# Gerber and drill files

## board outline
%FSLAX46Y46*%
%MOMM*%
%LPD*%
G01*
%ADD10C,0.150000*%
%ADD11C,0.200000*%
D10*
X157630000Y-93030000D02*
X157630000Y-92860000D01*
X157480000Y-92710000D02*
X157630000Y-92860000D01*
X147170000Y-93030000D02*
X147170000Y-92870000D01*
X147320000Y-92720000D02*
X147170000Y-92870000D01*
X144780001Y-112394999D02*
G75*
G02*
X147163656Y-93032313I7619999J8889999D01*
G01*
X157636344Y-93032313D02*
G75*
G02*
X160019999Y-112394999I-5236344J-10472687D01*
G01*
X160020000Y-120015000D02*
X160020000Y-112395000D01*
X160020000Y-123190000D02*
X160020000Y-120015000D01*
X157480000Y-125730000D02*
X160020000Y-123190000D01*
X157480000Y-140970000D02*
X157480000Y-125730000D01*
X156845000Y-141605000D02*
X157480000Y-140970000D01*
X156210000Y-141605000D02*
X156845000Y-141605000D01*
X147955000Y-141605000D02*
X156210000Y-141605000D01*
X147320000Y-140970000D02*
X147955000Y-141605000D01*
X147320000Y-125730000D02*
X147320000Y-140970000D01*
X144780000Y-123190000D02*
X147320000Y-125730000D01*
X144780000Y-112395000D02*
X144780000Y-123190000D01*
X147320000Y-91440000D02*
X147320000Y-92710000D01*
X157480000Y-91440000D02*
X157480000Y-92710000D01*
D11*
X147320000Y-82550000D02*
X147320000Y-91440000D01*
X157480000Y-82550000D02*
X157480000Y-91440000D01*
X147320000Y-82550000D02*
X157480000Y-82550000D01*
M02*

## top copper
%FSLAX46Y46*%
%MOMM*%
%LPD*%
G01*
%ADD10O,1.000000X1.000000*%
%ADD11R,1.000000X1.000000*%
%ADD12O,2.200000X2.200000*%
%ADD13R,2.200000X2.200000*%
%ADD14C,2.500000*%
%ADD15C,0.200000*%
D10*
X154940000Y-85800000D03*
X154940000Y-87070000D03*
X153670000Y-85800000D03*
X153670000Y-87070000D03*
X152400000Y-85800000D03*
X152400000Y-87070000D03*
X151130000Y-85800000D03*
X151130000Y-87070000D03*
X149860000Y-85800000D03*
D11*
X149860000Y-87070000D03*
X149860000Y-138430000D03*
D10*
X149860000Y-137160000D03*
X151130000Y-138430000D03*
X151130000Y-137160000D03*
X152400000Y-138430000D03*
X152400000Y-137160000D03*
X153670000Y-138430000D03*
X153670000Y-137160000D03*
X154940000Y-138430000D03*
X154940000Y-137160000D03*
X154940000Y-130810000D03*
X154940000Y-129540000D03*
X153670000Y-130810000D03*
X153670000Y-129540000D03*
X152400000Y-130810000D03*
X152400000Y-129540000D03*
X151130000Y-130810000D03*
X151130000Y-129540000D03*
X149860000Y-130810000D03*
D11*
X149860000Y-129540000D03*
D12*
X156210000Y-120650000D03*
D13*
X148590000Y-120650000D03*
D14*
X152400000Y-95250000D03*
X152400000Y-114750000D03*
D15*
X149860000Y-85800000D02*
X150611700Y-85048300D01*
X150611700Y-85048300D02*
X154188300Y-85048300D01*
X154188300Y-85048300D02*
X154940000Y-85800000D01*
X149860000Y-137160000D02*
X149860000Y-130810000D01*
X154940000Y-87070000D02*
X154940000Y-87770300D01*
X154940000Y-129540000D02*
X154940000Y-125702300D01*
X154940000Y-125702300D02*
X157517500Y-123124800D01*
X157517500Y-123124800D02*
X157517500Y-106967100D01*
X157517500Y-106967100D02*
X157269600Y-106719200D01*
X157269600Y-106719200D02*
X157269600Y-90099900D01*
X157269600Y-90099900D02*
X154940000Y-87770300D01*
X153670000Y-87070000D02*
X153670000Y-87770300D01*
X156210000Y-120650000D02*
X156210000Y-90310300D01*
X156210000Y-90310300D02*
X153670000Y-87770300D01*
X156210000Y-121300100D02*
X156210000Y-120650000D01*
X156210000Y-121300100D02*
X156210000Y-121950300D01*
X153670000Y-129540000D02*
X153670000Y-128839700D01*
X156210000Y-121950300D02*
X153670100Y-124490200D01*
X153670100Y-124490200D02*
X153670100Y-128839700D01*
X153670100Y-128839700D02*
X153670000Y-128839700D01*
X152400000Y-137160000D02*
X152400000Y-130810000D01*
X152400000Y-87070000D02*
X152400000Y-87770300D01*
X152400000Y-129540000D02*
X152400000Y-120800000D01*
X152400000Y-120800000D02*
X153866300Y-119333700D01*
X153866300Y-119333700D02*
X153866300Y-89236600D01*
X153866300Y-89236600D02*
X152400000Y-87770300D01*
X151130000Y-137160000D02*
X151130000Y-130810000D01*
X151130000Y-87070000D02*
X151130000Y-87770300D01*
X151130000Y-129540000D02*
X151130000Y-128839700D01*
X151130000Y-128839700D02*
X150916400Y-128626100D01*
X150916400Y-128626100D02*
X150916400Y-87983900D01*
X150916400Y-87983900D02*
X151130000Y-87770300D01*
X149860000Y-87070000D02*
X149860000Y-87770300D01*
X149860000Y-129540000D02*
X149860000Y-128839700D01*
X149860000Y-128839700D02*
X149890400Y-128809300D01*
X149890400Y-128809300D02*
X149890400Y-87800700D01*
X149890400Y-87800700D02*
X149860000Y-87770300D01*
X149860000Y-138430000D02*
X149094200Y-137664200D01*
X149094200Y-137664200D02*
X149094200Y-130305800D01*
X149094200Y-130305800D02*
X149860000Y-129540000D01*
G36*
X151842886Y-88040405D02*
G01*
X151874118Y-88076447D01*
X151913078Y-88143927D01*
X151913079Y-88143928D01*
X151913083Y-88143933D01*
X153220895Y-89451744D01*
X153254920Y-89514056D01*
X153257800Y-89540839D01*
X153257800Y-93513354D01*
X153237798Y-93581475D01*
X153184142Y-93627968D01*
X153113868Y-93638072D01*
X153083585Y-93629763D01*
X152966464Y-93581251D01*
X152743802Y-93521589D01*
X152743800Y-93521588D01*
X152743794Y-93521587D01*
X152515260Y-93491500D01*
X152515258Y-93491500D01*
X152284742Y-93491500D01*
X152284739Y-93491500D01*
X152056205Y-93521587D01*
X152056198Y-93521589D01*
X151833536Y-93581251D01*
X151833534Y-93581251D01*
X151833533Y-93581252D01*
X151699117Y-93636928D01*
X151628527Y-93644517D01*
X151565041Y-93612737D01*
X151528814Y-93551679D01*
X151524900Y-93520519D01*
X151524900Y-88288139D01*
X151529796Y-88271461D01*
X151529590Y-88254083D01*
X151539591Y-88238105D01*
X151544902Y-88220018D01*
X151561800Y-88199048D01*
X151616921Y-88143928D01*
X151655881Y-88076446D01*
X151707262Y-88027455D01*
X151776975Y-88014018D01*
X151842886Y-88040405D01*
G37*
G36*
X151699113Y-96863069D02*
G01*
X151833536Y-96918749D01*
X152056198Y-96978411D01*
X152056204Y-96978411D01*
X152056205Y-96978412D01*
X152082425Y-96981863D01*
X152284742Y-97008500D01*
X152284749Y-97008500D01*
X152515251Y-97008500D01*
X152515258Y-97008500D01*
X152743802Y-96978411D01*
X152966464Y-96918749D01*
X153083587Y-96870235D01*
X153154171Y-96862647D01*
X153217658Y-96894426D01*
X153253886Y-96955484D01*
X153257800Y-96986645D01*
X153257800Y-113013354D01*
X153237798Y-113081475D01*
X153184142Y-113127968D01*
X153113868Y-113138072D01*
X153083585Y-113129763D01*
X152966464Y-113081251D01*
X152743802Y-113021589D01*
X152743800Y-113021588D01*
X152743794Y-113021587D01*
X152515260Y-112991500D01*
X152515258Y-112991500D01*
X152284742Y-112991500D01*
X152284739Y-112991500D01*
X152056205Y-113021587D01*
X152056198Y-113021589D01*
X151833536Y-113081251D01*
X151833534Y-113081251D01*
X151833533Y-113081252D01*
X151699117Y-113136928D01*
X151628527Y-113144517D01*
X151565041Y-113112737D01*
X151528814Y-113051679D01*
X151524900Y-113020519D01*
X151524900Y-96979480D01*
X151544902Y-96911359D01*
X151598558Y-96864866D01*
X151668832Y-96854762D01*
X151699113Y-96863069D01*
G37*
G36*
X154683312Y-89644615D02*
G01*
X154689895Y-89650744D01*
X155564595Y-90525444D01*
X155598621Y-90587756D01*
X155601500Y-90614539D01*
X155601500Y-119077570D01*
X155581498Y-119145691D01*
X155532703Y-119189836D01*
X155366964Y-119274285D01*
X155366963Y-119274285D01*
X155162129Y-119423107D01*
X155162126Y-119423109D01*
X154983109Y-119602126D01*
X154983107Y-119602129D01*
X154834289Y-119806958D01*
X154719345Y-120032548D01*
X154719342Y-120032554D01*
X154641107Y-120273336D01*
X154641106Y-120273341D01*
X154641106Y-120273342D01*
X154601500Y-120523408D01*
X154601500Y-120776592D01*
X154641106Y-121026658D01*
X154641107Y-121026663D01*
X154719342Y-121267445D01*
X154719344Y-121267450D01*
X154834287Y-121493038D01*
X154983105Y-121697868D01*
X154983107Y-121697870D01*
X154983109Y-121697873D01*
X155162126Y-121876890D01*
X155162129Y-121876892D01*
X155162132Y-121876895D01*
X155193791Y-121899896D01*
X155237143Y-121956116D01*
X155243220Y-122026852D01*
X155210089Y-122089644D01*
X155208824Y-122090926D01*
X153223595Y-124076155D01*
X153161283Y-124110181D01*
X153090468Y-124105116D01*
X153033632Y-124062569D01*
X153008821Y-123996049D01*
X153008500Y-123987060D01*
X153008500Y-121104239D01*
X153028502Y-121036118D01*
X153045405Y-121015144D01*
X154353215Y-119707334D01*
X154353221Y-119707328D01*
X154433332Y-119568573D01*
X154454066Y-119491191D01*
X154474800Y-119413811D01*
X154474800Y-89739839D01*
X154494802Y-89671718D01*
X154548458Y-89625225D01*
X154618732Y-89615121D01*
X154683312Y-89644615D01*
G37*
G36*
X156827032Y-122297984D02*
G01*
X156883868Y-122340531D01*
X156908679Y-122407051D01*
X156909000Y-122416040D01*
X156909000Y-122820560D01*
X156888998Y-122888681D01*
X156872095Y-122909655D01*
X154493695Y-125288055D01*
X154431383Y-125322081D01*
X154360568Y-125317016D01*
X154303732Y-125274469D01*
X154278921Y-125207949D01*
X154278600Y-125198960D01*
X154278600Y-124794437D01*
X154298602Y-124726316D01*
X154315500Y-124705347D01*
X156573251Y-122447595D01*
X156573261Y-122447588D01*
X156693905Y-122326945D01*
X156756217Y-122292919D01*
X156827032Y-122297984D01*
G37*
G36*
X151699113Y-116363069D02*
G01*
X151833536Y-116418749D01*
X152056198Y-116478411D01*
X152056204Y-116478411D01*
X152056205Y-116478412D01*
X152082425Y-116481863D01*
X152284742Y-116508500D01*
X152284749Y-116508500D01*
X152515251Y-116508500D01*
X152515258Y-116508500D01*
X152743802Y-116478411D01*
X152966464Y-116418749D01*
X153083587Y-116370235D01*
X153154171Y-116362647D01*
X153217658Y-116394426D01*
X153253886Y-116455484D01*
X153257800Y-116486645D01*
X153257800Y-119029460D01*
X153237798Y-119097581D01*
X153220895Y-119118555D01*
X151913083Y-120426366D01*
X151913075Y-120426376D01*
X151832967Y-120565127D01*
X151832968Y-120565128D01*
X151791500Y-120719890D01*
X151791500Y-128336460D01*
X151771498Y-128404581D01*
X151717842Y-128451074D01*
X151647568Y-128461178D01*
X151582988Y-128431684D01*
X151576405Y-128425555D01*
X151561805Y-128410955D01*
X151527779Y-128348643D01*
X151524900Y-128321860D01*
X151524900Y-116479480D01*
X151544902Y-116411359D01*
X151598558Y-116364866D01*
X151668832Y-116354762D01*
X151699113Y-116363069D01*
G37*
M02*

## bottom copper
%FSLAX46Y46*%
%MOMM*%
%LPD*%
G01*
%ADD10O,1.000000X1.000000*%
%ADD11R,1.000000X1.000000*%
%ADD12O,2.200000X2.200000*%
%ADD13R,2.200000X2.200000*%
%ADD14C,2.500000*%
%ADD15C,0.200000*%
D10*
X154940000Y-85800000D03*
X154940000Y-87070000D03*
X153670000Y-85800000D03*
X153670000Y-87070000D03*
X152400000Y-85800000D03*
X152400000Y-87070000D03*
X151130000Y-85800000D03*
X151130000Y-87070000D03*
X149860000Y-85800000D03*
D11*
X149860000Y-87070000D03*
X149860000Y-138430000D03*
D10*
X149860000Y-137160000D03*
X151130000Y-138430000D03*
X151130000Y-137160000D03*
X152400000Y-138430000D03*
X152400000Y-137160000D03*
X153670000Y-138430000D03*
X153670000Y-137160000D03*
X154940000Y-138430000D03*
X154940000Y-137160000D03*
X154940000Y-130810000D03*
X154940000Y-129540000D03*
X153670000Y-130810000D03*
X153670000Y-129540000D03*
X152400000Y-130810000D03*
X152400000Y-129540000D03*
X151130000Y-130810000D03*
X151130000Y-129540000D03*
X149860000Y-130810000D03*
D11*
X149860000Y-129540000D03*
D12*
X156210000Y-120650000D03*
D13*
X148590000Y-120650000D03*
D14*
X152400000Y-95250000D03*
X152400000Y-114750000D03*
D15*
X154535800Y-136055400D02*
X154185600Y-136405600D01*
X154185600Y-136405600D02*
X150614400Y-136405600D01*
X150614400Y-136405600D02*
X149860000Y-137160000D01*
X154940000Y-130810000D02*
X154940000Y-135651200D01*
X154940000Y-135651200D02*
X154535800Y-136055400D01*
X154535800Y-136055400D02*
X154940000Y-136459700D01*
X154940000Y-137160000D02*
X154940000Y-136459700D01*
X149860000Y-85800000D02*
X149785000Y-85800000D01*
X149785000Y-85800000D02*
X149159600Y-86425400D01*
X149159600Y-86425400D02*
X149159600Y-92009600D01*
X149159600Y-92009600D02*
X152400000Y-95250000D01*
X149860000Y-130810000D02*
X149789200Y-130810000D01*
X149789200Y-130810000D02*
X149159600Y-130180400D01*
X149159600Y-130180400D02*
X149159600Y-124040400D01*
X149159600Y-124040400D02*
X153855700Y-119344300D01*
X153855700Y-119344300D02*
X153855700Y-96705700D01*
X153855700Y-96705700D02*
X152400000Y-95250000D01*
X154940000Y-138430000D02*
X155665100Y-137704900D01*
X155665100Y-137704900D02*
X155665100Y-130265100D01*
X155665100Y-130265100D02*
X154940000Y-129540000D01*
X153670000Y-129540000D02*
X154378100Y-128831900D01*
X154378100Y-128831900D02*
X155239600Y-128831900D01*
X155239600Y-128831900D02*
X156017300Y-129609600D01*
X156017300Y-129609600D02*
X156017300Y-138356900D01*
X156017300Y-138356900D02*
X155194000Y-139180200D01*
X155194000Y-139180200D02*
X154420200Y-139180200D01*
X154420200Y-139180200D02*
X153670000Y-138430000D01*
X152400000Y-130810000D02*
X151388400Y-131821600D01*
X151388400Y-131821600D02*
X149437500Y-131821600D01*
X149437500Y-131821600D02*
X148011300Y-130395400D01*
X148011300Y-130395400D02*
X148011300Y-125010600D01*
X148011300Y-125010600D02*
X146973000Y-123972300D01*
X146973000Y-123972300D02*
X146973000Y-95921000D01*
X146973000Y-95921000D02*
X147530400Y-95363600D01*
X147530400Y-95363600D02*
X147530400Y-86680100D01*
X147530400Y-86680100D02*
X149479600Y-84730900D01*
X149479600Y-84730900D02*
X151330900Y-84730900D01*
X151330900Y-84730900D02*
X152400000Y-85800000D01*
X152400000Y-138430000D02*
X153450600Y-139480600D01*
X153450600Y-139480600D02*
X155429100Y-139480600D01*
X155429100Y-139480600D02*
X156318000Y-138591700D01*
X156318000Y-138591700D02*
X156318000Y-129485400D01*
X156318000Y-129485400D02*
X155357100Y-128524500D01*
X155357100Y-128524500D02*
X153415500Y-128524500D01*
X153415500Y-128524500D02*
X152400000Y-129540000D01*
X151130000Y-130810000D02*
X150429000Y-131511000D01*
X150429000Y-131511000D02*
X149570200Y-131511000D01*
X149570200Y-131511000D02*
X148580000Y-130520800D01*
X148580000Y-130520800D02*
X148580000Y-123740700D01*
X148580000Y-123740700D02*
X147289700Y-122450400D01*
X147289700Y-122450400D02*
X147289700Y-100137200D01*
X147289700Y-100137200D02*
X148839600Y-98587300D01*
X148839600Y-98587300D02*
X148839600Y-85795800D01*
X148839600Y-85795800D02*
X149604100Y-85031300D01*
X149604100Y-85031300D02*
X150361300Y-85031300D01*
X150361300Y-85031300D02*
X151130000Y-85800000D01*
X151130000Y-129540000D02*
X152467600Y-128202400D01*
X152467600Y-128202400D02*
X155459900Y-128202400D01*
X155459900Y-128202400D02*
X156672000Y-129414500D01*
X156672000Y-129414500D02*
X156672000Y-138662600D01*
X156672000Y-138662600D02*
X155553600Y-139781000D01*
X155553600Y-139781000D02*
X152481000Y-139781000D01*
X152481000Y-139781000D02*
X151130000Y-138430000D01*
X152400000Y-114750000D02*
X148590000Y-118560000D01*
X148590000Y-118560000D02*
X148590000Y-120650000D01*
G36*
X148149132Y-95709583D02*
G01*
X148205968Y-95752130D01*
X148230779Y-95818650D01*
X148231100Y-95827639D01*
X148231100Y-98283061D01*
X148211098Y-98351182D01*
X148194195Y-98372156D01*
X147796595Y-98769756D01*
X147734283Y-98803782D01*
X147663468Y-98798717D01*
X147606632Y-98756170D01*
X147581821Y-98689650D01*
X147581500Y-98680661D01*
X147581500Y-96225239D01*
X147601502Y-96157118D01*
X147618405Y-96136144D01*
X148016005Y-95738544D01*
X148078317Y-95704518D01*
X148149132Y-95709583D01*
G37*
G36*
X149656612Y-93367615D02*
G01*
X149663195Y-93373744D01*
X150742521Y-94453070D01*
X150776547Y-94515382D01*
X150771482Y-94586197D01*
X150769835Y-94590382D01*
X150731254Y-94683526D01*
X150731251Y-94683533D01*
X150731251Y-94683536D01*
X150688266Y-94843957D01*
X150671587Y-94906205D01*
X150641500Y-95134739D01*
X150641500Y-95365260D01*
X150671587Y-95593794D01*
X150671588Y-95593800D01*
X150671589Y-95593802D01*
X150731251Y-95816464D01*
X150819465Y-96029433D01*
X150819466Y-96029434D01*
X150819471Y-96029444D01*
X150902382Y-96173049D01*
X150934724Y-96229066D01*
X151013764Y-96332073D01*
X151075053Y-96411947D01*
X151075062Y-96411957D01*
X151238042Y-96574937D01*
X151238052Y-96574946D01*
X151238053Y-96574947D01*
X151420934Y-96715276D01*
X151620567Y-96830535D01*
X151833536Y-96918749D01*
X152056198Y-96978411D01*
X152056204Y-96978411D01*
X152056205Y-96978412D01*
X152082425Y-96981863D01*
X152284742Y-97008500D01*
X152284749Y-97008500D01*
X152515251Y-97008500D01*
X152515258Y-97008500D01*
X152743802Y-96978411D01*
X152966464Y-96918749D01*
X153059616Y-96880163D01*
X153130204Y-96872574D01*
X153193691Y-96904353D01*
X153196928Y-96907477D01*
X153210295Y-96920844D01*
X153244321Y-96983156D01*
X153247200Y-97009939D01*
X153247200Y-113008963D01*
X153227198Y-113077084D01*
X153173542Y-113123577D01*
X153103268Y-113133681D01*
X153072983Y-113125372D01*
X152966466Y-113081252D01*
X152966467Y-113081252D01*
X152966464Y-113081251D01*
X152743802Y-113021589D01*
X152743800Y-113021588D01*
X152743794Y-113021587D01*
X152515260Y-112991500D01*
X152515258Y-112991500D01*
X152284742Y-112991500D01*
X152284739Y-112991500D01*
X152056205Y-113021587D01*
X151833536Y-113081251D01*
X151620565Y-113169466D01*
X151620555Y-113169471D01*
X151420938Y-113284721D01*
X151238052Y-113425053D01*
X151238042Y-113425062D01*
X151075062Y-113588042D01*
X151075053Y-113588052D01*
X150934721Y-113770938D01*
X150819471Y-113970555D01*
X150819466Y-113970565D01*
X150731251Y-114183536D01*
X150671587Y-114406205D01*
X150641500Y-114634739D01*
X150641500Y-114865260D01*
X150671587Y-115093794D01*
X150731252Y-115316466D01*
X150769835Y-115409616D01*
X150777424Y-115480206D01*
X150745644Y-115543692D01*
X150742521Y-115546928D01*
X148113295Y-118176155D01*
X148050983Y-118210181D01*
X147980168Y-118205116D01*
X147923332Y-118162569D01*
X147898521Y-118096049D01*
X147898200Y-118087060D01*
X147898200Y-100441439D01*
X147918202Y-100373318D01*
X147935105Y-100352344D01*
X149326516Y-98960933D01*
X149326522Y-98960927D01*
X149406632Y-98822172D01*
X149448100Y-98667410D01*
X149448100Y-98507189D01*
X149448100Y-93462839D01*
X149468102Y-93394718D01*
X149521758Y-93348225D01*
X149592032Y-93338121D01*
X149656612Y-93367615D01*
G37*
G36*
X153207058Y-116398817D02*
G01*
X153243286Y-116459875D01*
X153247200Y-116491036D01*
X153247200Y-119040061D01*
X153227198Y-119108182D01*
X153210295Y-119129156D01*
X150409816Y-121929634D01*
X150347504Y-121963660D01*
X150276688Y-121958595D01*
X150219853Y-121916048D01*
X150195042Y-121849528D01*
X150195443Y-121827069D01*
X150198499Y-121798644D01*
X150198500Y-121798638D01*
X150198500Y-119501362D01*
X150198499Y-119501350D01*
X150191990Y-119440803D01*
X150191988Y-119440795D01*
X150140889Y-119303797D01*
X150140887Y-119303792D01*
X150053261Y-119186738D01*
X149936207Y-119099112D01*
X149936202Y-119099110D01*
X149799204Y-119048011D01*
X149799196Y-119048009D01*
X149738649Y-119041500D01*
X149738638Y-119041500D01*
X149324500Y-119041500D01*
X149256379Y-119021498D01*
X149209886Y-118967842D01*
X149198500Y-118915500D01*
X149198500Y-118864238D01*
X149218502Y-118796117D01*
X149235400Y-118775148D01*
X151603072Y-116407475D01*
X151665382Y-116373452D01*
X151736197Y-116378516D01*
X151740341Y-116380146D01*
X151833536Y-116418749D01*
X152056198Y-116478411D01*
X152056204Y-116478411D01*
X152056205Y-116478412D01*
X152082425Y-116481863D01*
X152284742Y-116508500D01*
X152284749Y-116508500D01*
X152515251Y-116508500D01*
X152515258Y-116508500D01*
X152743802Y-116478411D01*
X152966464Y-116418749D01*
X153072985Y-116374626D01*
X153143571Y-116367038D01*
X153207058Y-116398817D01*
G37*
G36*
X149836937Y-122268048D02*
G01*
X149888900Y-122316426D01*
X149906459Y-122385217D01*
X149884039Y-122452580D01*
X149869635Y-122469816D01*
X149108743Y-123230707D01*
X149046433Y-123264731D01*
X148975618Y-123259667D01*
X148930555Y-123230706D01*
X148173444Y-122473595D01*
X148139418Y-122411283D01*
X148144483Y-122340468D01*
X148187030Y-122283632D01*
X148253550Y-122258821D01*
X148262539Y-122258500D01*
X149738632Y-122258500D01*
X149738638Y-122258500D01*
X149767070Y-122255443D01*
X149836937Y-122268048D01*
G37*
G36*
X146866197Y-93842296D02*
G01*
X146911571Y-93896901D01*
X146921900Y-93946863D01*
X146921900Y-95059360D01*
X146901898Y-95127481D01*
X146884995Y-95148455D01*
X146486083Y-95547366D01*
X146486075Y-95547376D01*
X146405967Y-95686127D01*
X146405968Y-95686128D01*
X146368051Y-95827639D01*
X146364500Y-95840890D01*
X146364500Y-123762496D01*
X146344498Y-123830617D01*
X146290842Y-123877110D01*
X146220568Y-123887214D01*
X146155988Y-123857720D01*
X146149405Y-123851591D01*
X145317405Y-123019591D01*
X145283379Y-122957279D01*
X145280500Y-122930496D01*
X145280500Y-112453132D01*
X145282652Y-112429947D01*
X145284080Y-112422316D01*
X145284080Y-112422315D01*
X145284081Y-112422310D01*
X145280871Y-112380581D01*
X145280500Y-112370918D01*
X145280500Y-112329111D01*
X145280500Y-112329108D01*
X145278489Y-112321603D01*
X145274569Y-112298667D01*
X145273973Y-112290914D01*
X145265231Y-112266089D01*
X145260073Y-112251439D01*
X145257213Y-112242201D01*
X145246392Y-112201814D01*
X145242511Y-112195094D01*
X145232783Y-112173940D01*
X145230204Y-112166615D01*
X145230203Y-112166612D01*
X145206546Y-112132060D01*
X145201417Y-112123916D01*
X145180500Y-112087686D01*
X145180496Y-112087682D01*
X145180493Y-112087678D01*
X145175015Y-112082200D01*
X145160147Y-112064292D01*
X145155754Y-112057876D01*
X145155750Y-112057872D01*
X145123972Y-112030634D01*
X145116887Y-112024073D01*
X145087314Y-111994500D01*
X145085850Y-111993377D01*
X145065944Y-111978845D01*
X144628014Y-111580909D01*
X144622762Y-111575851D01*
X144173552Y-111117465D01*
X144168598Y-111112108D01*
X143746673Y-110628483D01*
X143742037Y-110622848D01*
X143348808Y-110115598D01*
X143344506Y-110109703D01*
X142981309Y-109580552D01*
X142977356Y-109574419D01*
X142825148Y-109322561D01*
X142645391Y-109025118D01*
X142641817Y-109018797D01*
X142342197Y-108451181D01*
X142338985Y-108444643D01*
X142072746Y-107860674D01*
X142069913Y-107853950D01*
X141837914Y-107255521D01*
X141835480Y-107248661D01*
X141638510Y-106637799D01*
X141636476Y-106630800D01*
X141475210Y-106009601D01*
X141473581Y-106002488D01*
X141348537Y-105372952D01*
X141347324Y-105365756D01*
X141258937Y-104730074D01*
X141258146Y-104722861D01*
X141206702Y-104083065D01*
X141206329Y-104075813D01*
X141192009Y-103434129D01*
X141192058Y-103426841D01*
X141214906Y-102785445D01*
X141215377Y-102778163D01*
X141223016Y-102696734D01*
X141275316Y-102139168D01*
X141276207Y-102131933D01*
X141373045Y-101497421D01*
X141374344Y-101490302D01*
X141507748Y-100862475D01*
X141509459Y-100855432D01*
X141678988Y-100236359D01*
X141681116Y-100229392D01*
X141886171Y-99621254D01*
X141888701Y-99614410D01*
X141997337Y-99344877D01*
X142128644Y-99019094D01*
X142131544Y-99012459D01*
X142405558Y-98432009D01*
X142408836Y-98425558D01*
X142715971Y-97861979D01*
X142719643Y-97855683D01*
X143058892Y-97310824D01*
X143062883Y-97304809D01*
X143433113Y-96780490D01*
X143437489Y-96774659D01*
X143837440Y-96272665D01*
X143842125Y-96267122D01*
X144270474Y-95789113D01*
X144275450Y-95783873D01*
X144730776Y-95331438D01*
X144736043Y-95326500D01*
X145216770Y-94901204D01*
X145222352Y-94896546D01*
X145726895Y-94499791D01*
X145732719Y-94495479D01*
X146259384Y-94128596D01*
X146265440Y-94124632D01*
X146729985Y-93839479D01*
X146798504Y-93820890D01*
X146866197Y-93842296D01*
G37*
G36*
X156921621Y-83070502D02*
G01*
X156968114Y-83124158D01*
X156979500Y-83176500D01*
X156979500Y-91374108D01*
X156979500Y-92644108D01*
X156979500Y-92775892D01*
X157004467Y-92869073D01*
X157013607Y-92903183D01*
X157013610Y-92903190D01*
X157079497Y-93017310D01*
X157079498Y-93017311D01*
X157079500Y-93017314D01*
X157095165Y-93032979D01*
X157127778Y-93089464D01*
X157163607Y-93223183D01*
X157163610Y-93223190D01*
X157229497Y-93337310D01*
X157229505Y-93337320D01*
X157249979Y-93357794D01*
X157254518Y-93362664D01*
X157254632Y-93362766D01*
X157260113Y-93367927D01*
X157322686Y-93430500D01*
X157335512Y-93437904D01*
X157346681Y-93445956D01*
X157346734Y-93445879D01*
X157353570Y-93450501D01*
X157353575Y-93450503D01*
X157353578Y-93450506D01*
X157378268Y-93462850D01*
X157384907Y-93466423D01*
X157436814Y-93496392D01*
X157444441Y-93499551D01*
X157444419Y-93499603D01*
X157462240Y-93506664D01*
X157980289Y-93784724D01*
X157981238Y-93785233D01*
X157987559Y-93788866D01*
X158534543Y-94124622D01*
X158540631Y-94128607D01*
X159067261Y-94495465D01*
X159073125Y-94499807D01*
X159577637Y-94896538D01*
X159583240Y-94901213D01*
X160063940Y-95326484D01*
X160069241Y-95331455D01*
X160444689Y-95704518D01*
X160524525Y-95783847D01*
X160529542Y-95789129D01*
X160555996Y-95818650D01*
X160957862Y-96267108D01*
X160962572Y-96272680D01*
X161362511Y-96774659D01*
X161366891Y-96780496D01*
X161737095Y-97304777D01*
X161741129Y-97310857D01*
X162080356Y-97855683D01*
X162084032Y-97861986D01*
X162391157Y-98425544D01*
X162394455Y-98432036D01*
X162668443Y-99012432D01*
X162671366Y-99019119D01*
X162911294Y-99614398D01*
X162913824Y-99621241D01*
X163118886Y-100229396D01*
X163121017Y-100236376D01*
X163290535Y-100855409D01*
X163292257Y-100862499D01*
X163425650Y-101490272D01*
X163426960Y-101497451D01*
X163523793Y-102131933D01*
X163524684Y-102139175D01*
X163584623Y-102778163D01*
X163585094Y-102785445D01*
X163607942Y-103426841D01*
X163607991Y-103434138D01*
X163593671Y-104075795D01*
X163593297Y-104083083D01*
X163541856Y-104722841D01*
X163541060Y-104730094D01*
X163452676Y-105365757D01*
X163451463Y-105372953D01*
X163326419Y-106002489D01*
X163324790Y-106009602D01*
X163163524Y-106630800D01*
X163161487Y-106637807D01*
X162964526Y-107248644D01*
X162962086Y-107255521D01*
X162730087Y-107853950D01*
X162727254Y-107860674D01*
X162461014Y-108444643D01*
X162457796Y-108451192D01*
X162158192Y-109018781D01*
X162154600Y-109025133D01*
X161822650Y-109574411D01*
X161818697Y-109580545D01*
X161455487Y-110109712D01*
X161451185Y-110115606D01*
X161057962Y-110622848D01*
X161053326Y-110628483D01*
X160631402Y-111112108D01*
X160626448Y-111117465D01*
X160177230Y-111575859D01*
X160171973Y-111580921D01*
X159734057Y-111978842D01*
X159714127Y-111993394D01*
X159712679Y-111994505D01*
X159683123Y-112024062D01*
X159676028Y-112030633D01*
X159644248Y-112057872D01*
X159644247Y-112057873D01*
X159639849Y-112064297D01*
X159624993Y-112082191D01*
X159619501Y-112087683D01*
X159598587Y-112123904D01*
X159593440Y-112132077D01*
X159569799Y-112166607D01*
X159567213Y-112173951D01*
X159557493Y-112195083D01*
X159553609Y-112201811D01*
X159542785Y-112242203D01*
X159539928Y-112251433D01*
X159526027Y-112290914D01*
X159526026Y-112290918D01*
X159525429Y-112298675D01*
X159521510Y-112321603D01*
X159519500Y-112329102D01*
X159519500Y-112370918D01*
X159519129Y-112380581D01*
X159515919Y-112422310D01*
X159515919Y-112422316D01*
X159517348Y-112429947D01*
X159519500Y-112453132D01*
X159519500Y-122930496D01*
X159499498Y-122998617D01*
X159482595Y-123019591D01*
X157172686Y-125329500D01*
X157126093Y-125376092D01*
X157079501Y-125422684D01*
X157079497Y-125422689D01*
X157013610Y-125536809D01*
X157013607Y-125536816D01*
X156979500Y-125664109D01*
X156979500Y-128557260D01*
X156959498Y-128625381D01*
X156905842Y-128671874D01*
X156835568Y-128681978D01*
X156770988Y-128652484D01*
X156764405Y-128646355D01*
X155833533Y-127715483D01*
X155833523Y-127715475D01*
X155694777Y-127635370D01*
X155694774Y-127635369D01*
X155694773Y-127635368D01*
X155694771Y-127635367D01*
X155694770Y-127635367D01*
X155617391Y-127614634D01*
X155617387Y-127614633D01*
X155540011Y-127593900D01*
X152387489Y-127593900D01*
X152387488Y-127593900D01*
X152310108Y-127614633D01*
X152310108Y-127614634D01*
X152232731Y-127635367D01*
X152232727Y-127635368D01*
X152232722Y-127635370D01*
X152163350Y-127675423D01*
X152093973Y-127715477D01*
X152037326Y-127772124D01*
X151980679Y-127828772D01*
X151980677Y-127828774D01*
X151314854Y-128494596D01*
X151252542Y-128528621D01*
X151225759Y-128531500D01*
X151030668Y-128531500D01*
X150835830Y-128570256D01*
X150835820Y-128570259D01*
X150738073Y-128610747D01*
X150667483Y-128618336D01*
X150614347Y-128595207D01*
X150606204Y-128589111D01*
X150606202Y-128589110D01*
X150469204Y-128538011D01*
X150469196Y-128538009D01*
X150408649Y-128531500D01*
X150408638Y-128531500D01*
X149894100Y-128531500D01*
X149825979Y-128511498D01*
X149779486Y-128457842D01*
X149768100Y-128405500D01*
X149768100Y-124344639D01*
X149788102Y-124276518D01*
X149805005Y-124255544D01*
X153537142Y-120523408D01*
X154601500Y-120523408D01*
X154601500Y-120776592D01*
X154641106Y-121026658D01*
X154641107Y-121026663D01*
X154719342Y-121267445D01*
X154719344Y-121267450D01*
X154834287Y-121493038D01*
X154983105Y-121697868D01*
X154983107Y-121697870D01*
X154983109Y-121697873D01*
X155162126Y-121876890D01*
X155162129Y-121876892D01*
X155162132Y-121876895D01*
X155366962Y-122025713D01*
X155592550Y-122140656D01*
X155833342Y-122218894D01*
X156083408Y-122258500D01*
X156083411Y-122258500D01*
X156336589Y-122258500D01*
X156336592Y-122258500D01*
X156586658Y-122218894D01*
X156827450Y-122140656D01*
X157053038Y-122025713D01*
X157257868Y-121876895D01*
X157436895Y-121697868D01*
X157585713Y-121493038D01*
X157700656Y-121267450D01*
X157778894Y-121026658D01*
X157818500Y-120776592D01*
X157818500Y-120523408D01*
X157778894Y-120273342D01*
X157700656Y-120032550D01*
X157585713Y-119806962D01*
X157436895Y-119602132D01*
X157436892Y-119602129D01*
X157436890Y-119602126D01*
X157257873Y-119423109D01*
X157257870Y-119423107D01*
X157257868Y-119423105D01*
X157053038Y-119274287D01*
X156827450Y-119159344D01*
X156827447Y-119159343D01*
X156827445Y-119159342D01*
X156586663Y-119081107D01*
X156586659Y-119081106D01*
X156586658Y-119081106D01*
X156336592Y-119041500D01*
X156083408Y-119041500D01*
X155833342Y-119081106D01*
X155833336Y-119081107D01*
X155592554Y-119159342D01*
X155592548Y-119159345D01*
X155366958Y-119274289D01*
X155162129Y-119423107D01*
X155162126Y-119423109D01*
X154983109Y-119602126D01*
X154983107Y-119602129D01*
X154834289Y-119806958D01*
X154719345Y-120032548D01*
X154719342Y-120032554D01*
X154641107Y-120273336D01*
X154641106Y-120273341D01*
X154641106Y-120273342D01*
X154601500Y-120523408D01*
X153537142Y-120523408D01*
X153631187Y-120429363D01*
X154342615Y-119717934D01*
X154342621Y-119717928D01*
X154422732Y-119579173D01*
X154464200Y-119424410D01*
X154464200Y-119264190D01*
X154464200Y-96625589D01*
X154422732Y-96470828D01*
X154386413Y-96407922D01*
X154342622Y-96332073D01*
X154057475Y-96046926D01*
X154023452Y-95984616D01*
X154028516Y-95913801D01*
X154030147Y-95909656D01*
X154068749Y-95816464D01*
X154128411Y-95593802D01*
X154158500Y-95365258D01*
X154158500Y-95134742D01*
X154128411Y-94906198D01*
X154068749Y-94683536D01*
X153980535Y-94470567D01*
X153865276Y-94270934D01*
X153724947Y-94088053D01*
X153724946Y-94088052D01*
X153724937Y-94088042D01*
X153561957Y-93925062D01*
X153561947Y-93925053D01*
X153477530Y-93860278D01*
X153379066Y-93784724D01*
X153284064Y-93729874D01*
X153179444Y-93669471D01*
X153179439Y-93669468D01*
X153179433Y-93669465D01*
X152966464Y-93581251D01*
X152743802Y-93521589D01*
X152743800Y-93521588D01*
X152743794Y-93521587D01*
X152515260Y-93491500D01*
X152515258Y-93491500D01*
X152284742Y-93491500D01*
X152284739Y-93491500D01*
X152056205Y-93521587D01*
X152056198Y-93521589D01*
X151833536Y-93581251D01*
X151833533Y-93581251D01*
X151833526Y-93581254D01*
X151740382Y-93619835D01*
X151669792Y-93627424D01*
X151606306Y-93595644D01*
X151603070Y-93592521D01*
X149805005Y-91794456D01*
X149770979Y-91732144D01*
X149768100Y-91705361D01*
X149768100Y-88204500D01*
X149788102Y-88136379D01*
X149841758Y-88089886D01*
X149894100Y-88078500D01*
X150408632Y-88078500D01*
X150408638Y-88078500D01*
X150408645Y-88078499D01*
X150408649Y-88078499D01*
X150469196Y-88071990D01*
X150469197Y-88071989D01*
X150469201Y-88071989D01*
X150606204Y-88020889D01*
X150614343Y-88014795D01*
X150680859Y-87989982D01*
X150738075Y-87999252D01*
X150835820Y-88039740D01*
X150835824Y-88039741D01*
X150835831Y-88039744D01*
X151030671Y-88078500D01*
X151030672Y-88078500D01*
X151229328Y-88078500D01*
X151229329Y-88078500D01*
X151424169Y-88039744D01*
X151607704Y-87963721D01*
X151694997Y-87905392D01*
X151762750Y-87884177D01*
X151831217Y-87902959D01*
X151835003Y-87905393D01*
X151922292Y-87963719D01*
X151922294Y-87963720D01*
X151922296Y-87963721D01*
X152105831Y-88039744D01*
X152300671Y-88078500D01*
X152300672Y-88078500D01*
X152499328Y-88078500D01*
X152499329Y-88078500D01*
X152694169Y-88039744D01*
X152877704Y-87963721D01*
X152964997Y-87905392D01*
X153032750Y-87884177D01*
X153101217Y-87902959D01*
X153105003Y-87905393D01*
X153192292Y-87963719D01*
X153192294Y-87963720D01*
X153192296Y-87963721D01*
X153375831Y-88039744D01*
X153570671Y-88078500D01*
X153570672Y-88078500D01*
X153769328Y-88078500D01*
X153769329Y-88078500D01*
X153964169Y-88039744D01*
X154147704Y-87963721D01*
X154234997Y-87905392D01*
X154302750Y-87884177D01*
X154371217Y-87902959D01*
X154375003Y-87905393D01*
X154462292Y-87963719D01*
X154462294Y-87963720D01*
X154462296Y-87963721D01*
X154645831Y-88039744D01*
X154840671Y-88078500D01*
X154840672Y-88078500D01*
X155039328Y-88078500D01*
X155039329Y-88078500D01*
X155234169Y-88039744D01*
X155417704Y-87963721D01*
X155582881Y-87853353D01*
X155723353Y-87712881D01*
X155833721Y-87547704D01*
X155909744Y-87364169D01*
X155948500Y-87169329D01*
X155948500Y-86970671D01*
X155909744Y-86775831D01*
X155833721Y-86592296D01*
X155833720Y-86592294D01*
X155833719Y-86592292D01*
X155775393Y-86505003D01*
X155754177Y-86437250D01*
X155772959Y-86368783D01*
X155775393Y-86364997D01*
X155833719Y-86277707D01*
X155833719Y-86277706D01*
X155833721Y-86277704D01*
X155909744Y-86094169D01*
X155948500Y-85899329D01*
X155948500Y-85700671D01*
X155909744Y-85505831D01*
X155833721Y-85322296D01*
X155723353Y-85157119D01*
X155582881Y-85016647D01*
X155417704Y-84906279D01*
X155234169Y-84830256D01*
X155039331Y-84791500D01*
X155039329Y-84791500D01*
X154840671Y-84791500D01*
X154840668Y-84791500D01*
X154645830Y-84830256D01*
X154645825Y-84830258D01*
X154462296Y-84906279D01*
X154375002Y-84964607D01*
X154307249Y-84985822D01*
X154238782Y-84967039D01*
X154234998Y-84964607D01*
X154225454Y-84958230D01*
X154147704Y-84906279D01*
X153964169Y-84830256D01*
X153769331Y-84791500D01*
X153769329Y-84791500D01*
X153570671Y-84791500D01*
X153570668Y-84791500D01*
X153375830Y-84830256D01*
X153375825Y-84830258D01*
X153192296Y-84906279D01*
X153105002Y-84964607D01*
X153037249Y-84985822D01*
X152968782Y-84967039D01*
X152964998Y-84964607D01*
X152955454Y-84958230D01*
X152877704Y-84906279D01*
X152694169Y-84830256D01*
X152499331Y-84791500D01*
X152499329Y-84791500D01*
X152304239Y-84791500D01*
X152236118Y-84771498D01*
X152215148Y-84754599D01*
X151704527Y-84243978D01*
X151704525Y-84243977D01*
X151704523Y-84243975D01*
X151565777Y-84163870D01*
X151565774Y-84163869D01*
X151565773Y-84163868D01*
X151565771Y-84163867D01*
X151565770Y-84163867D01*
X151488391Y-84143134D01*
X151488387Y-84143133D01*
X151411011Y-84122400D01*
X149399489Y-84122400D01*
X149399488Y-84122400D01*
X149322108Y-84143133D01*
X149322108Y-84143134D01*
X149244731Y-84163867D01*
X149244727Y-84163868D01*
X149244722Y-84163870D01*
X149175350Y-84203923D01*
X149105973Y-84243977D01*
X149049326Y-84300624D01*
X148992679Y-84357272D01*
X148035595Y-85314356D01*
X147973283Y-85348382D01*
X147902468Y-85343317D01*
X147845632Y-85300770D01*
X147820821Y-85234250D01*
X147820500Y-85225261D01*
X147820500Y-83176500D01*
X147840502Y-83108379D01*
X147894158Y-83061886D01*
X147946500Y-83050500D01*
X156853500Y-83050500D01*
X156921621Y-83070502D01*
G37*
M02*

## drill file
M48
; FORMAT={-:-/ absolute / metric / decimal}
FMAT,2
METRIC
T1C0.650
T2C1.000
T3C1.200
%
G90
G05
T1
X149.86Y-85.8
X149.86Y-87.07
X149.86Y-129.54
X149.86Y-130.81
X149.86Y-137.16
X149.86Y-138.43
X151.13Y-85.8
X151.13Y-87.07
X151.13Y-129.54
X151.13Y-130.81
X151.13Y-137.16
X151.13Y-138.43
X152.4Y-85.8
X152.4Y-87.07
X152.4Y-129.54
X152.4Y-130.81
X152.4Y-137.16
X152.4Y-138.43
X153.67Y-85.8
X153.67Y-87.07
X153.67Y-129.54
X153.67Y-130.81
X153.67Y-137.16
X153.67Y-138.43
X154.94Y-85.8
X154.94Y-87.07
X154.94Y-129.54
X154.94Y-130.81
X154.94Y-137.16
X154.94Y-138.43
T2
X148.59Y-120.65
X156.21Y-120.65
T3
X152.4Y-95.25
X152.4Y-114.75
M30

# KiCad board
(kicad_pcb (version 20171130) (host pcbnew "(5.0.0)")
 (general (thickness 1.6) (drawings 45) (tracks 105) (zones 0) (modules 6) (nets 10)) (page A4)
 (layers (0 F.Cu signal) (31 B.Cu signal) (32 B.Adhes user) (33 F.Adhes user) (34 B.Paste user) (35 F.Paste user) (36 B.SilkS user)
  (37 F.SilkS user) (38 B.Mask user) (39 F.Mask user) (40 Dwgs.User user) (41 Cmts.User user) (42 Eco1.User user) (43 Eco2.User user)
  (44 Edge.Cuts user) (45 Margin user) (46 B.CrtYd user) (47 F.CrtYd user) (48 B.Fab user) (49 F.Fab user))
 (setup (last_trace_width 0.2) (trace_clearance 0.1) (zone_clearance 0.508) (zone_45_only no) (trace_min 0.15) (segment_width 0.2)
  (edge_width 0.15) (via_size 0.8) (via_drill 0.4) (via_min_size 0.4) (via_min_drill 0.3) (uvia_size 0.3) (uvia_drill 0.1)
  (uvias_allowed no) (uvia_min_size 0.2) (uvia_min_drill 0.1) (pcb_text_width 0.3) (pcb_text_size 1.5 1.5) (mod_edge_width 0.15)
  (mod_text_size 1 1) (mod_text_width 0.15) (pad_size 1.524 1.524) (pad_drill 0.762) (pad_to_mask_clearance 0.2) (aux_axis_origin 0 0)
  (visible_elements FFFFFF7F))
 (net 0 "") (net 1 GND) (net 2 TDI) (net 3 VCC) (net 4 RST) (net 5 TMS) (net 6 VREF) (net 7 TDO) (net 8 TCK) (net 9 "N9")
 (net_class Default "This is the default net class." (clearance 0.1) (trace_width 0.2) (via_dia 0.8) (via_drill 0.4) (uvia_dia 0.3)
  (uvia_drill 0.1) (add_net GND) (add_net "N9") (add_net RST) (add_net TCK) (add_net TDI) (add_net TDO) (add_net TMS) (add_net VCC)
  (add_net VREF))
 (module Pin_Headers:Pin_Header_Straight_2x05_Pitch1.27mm (layer F.Cu) (at 149.86 87.07 90)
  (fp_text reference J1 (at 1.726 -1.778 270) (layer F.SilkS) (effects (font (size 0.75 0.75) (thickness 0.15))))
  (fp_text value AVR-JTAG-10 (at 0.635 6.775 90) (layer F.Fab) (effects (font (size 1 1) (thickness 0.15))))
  (pad 10 thru_hole oval (at 1.27 5.08 90) (size 1 1) (drill 0.65) (layers *.Cu *.Mask) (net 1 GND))
  (pad 9 thru_hole oval (at 0 5.08 90) (size 1 1) (drill 0.65) (layers *.Cu *.Mask) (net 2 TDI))
  (pad 8 thru_hole oval (at 1.27 3.81 90) (size 1 1) (drill 0.65) (layers *.Cu *.Mask))
  (pad 7 thru_hole oval (at 0 3.81 90) (size 1 1) (drill 0.65) (layers *.Cu *.Mask) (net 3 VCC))
  (pad 6 thru_hole oval (at 1.27 2.54 90) (size 1 1) (drill 0.65) (layers *.Cu *.Mask) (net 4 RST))
  (pad 5 thru_hole oval (at 0 2.54 90) (size 1 1) (drill 0.65) (layers *.Cu *.Mask) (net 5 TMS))
  (pad 4 thru_hole oval (at 1.27 1.27 90) (size 1 1) (drill 0.65) (layers *.Cu *.Mask) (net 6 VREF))
  (pad 3 thru_hole oval (at 0 1.27 90) (size 1 1) (drill 0.65) (layers *.Cu *.Mask) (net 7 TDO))
  (pad 2 thru_hole oval (at 1.27 0 90) (size 1 1) (drill 0.65) (layers *.Cu *.Mask) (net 1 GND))
  (pad 1 thru_hole rect (at 0 0 90) (size 1 1) (drill 0.65) (layers *.Cu *.Mask) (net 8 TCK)))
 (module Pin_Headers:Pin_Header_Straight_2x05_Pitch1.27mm (layer F.Cu) (at 149.86 138.43 90)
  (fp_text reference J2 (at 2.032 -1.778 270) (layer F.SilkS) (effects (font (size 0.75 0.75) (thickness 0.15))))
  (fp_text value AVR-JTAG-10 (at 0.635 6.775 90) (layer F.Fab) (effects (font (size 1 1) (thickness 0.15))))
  (pad 1 thru_hole rect (at 0 0 90) (size 1 1) (drill 0.65) (layers *.Cu *.Mask) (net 8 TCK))
  (pad 2 thru_hole oval (at 1.27 0 90) (size 1 1) (drill 0.65) (layers *.Cu *.Mask) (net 1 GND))
  (pad 3 thru_hole oval (at 0 1.27 90) (size 1 1) (drill 0.65) (layers *.Cu *.Mask) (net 7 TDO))
  (pad 4 thru_hole oval (at 1.27 1.27 90) (size 1 1) (drill 0.65) (layers *.Cu *.Mask) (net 6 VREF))
  (pad 5 thru_hole oval (at 0 2.54 90) (size 1 1) (drill 0.65) (layers *.Cu *.Mask) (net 5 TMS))
  (pad 6 thru_hole oval (at 1.27 2.54 90) (size 1 1) (drill 0.65) (layers *.Cu *.Mask) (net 4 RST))
  (pad 7 thru_hole oval (at 0 3.81 90) (size 1 1) (drill 0.65) (layers *.Cu *.Mask) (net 3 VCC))
  (pad 8 thru_hole oval (at 1.27 3.81 90) (size 1 1) (drill 0.65) (layers *.Cu *.Mask))
  (pad 9 thru_hole oval (at 0 5.08 90) (size 1 1) (drill 0.65) (layers *.Cu *.Mask) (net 2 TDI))
  (pad 10 thru_hole oval (at 1.27 5.08 90) (size 1 1) (drill 0.65) (layers *.Cu *.Mask) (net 1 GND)))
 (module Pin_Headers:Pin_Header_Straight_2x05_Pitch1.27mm (layer B.Cu) (at 149.86 129.54 270)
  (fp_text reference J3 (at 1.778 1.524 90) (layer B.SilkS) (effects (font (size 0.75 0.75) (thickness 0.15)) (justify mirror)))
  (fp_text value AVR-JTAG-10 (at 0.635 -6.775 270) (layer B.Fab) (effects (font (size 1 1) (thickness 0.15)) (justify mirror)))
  (pad 10 thru_hole oval (at 1.27 -5.08 270) (size 1 1) (drill 0.65) (layers *.Cu *.Mask) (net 1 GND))
  (pad 9 thru_hole oval (at 0 -5.08 270) (size 1 1) (drill 0.65) (layers *.Cu *.Mask) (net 2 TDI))
  (pad 8 thru_hole oval (at 1.27 -3.81 270) (size 1 1) (drill 0.65) (layers *.Cu *.Mask))
  (pad 7 thru_hole oval (at 0 -3.81 270) (size 1 1) (drill 0.65) (layers *.Cu *.Mask) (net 3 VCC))
  (pad 6 thru_hole oval (at 1.27 -2.54 270) (size 1 1) (drill 0.65) (layers *.Cu *.Mask) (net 4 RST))
  (pad 5 thru_hole oval (at 0 -2.54 270) (size 1 1) (drill 0.65) (layers *.Cu *.Mask) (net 5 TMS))
  (pad 4 thru_hole oval (at 1.27 -1.27 270) (size 1 1) (drill 0.65) (layers *.Cu *.Mask) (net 6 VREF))
  (pad 3 thru_hole oval (at 0 -1.27 270) (size 1 1) (drill 0.65) (layers *.Cu *.Mask) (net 7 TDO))
  (pad 2 thru_hole oval (at 1.27 0 270) (size 1 1) (drill 0.65) (layers *.Cu *.Mask) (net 1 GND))
  (pad 1 thru_hole rect (at 0 0 270) (size 1 1) (drill 0.65) (layers *.Cu *.Mask) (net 8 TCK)))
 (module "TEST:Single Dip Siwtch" (layer F.Cu) (at 148.59 120.65 90)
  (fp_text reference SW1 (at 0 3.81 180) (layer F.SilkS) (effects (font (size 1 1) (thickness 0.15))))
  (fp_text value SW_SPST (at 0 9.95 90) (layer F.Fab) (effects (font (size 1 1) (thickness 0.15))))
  (pad 2 thru_hole oval (at 0 7.62 90) (size 2.2 2.2) (drill 1) (layers *.Cu *.Mask) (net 3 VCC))
  (pad 1 thru_hole rect (at 0 0 90) (size 2.2 2.2) (drill 1) (layers *.Cu *.Mask) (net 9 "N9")))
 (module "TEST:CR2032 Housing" (layer F.Cu) (at 152.4 103.25)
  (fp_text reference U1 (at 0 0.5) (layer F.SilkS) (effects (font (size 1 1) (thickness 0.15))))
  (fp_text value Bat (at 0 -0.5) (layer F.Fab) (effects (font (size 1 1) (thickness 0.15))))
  (pad 1 thru_hole circle (at 0 -8) (size 2.5 2.5) (drill 1.2) (layers *.Cu *.Mask) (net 1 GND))
  (pad 2 thru_hole circle (at 0 11.5) (size 2.5 2.5) (drill 1.2) (layers *.Cu *.Mask) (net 9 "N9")))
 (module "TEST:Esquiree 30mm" (layer B.Cu) (at 147.32 104.775 270)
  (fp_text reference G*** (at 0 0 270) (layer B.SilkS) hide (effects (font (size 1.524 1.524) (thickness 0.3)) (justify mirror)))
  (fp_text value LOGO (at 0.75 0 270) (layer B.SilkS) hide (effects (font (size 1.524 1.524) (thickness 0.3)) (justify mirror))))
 (gr_line (start 157.63 93.03) (end 157.63 92.86) (layer Edge.Cuts) (width 0.15))
 (gr_line (start 157.48 92.71) (end 157.63 92.86) (layer Edge.Cuts) (width 0.15))
 (gr_line (start 147.17 93.03) (end 147.17 92.87) (layer Edge.Cuts) (width 0.15))
 (gr_line (start 147.32 92.72) (end 147.17 92.87) (layer Edge.Cuts) (width 0.15))
 (gr_arc (start 152.4 103.505) (end 144.780001 112.394999) (angle 112.8336542) (layer Edge.Cuts) (width 0.15))
 (gr_arc (start 152.4 103.505) (end 160.019999 112.394999) (angle -112.8336542) (layer Edge.Cuts) (width 0.15))
 (gr_line (start 160.02 120.015) (end 160.02 112.395) (layer Edge.Cuts) (width 0.15))
 (gr_line (start 160.02 123.19) (end 160.02 120.015) (layer Edge.Cuts) (width 0.15))
 (gr_line (start 157.48 125.73) (end 160.02 123.19) (layer Edge.Cuts) (width 0.15))
 (gr_line (start 157.48 140.97) (end 157.48 125.73) (layer Edge.Cuts) (width 0.15))
 (gr_line (start 156.845 141.605) (end 157.48 140.97) (layer Edge.Cuts) (width 0.15))
 (gr_line (start 156.21 141.605) (end 156.845 141.605) (layer Edge.Cuts) (width 0.15))
 (gr_line (start 147.955 141.605) (end 156.21 141.605) (layer Edge.Cuts) (width 0.15))
 (gr_line (start 147.32 140.97) (end 147.955 141.605) (layer Edge.Cuts) (width 0.15))
 (gr_line (start 147.32 125.73) (end 147.32 140.97) (layer Edge.Cuts) (width 0.15))
 (gr_line (start 144.78 123.19) (end 147.32 125.73) (layer Edge.Cuts) (width 0.15))
 (gr_line (start 144.78 112.395) (end 144.78 123.19) (layer Edge.Cuts) (width 0.15))
 (gr_line (start 147.32 91.44) (end 147.32 92.71) (layer Edge.Cuts) (width 0.15))
 (gr_line (start 157.48 91.44) (end 157.48 92.71) (layer Edge.Cuts) (width 0.15))
 (gr_line (start 147.32 82.55) (end 147.32 91.44) (layer Edge.Cuts) (width 0.2))
 (gr_line (start 157.48 82.55) (end 157.48 91.44) (layer Edge.Cuts) (width 0.2))
 (gr_line (start 147.32 82.55) (end 157.48 82.55) (layer Edge.Cuts) (width 0.2))
 (segment (start 154.5358 136.0554) (end 154.1856 136.4056) (width 0.2) (layer B.Cu) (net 1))
 (segment (start 154.1856 136.4056) (end 150.6144 136.4056) (width 0.2) (layer B.Cu) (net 1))
 (segment (start 150.6144 136.4056) (end 149.86 137.16) (width 0.2) (layer B.Cu) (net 1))
 (segment (start 154.94 130.81) (end 154.94 135.6512) (width 0.2) (layer B.Cu) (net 1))
 (segment (start 154.94 135.6512) (end 154.5358 136.0554) (width 0.2) (layer B.Cu) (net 1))
 (segment (start 154.5358 136.0554) (end 154.94 136.4597) (width 0.2) (layer B.Cu) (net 1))
 (segment (start 154.94 137.16) (end 154.94 136.4597) (width 0.2) (layer B.Cu) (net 1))
 (segment (start 149.86 85.8) (end 149.785 85.8) (width 0.2) (layer B.Cu) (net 1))
 (segment (start 149.785 85.8) (end 149.1596 86.4254) (width 0.2) (layer B.Cu) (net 1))
 (segment (start 149.1596 86.4254) (end 149.1596 92.0096) (width 0.2) (layer B.Cu) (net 1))
 (segment (start 149.1596 92.0096) (end 152.4 95.25) (width 0.2) (layer B.Cu) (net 1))
 (segment (start 149.86 85.8) (end 150.6117 85.0483) (width 0.2) (layer F.Cu) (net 1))
 (segment (start 150.6117 85.0483) (end 154.1883 85.0483) (width 0.2) (layer F.Cu) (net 1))
 (segment (start 154.1883 85.0483) (end 154.94 85.8) (width 0.2) (layer F.Cu) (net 1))
 (segment (start 149.86 130.81) (end 149.7892 130.81) (width 0.2) (layer B.Cu) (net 1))
 (segment (start 149.7892 130.81) (end 149.1596 130.1804) (width 0.2) (layer B.Cu) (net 1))
 (segment (start 149.1596 130.1804) (end 149.1596 124.0404) (width 0.2) (layer B.Cu) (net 1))
 (segment (start 149.1596 124.0404) (end 153.8557 119.3443) (width 0.2) (layer B.Cu) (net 1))
 (segment (start 153.8557 119.3443) (end 153.8557 96.7057) (width 0.2) (layer B.Cu) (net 1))
 (segment (start 153.8557 96.7057) (end 152.4 95.25) (width 0.2) (layer B.Cu) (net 1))
 (segment (start 149.86 137.16) (end 149.86 130.81) (width 0.2) (layer F.Cu) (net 1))
 (segment (start 154.94 138.43) (end 155.6651 137.7049) (width 0.2) (layer B.Cu) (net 2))
 (segment (start 155.6651 137.7049) (end 155.6651 130.2651) (width 0.2) (layer B.Cu) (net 2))
 (segment (start 155.6651 130.2651) (end 154.94 129.54) (width 0.2) (layer B.Cu) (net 2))
 (segment (start 154.94 87.07) (end 154.94 87.7703) (width 0.2) (layer F.Cu) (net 2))
 (segment (start 154.94 129.54) (end 154.94 125.7023) (width 0.2) (layer F.Cu) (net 2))
 (segment (start 154.94 125.7023) (end 157.5175 123.1248) (width 0.2) (layer F.Cu) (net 2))
 (segment (start 157.5175 123.1248) (end 157.5175 106.9671) (width 0.2) (layer F.Cu) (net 2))
 (segment (start 157.5175 106.9671) (end 157.2696 106.7192) (width 0.2) (layer F.Cu) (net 2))
 (segment (start 157.2696 106.7192) (end 157.2696 90.0999) (width 0.2) (layer F.Cu) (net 2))
 (segment (start 157.2696 90.0999) (end 154.94 87.7703) (width 0.2) (layer F.Cu) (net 2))
 (segment (start 153.67 87.07) (end 153.67 87.7703) (width 0.2) (layer F.Cu) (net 3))
 (segment (start 156.21 120.65) (end 156.21 90.3103) (width 0.2) (layer F.Cu) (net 3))
 (segment (start 156.21 90.3103) (end 153.67 87.7703) (width 0.2) (layer F.Cu) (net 3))
 (segment (start 156.21 121.3001) (end 156.21 120.65) (width 0.2) (layer F.Cu) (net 3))
 (segment (start 153.67 129.54) (end 154.3781 128.8319) (width 0.2) (layer B.Cu) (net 3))
 (segment (start 154.3781 128.8319) (end 155.2396 128.8319) (width 0.2) (layer B.Cu) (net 3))
 (segment (start 155.2396 128.8319) (end 156.0173 129.6096) (width 0.2) (layer B.Cu) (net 3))
 (segment (start 156.0173 129.6096) (end 156.0173 138.3569) (width 0.2) (layer B.Cu) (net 3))
 (segment (start 156.0173 138.3569) (end 155.194 139.1802) (width 0.2) (layer B.Cu) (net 3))
 (segment (start 155.194 139.1802) (end 154.4202 139.1802) (width 0.2) (layer B.Cu) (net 3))
 (segment (start 154.4202 139.1802) (end 153.67 138.43) (width 0.2) (layer B.Cu) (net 3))
 (segment (start 156.21 121.3001) (end 156.21 121.9503) (width 0.2) (layer F.Cu) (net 3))
 (segment (start 153.67 129.54) (end 153.67 128.8397) (width 0.2) (layer F.Cu) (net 3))
 (segment (start 156.21 121.9503) (end 153.6701 124.4902) (width 0.2) (layer F.Cu) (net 3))
 (segment (start 153.6701 124.4902) (end 153.6701 128.8397) (width 0.2) (layer F.Cu) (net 3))
 (segment (start 153.6701 128.8397) (end 153.67 128.8397) (width 0.2) (layer F.Cu) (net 3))
 (segment (start 152.4 130.81) (end 151.3884 131.8216) (width 0.2) (layer B.Cu) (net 4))
 (segment (start 151.3884 131.8216) (end 149.4375 131.8216) (width 0.2) (layer B.Cu) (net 4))
 (segment (start 149.4375 131.8216) (end 148.0113 130.3954) (width 0.2) (layer B.Cu) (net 4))
 (segment (start 148.0113 130.3954) (end 148.0113 125.0106) (width 0.2) (layer B.Cu) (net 4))
 (segment (start 148.0113 125.0106) (end 146.973 123.9723) (width 0.2) (layer B.Cu) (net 4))
 (segment (start 146.973 123.9723) (end 146.973 95.921) (width 0.2) (layer B.Cu) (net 4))
 (segment (start 146.973 95.921) (end 147.5304 95.3636) (width 0.2) (layer B.Cu) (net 4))
 (segment (start 147.5304 95.3636) (end 147.5304 86.6801) (width 0.2) (layer B.Cu) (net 4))
 (segment (start 147.5304 86.6801) (end 149.4796 84.7309) (width 0.2) (layer B.Cu) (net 4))
 (segment (start 149.4796 84.7309) (end 151.3309 84.7309) (width 0.2) (layer B.Cu) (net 4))
 (segment (start 151.3309 84.7309) (end 152.4 85.8) (width 0.2) (layer B.Cu) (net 4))
 (segment (start 152.4 137.16) (end 152.4 130.81) (width 0.2) (layer F.Cu) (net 4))
 (segment (start 152.4 138.43) (end 153.4506 139.4806) (width 0.2) (layer B.Cu) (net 5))
 (segment (start 153.4506 139.4806) (end 155.4291 139.4806) (width 0.2) (layer B.Cu) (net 5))
 (segment (start 155.4291 139.4806) (end 156.318 138.5917) (width 0.2) (layer B.Cu) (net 5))
 (segment (start 156.318 138.5917) (end 156.318 129.4854) (width 0.2) (layer B.Cu) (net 5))
 (segment (start 156.318 129.4854) (end 155.3571 128.5245) (width 0.2) (layer B.Cu) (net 5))
 (segment (start 155.3571 128.5245) (end 153.4155 128.5245) (width 0.2) (layer B.Cu) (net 5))
 (segment (start 153.4155 128.5245) (end 152.4 129.54) (width 0.2) (layer B.Cu) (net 5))
 (segment (start 152.4 87.07) (end 152.4 87.7703) (width 0.2) (layer F.Cu) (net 5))
 (segment (start 152.4 129.54) (end 152.4 120.8) (width 0.2) (layer F.Cu) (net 5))
 (segment (start 152.4 120.8) (end 153.8663 119.3337) (width 0.2) (layer F.Cu) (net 5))
 (segment (start 153.8663 119.3337) (end 153.8663 89.2366) (width 0.2) (layer F.Cu) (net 5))
 (segment (start 153.8663 89.2366) (end 152.4 87.7703) (width 0.2) (layer F.Cu) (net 5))
 (segment (start 151.13 130.81) (end 150.429 131.511) (width 0.2) (layer B.Cu) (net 6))
 (segment (start 150.429 131.511) (end 149.5702 131.511) (width 0.2) (layer B.Cu) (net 6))
 (segment (start 149.5702 131.511) (end 148.58 130.5208) (width 0.2) (layer B.Cu) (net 6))
 (segment (start 148.58 130.5208) (end 148.58 123.7407) (width 0.2) (layer B.Cu) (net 6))
 (segment (start 148.58 123.7407) (end 147.2897 122.4504) (width 0.2) (layer B.Cu) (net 6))
 (segment (start 147.2897 122.4504) (end 147.2897 100.1372) (width 0.2) (layer B.Cu) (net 6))
 (segment (start 147.2897 100.1372) (end 148.8396 98.5873) (width 0.2) (layer B.Cu) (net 6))
 (segment (start 148.8396 98.5873) (end 148.8396 85.7958) (width 0.2) (layer B.Cu) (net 6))
 (segment (start 148.8396 85.7958) (end 149.6041 85.0313) (width 0.2) (layer B.Cu) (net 6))
 (segment (start 149.6041 85.0313) (end 150.3613 85.0313) (width 0.2) (layer B.Cu) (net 6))
 (segment (start 150.3613 85.0313) (end 151.13 85.8) (width 0.2) (layer B.Cu) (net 6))
 (segment (start 151.13 137.16) (end 151.13 130.81) (width 0.2) (layer F.Cu) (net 6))
 (segment (start 151.13 87.07) (end 151.13 87.7703) (width 0.2) (layer F.Cu) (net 7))
 (segment (start 151.13 129.54) (end 151.13 128.8397) (width 0.2) (layer F.Cu) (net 7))
 (segment (start 151.13 128.8397) (end 150.9164 128.6261) (width 0.2) (layer F.Cu) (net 7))
 (segment (start 150.9164 128.6261) (end 150.9164 87.9839) (width 0.2) (layer F.Cu) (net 7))
 (segment (start 150.9164 87.9839) (end 151.13 87.7703) (width 0.2) (layer F.Cu) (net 7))
 (segment (start 151.13 129.54) (end 152.4676 128.2024) (width 0.2) (layer B.Cu) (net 7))
 (segment (start 152.4676 128.2024) (end 155.4599 128.2024) (width 0.2) (layer B.Cu) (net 7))
 (segment (start 155.4599 128.2024) (end 156.672 129.4145) (width 0.2) (layer B.Cu) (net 7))
 (segment (start 156.672 129.4145) (end 156.672 138.6626) (width 0.2) (layer B.Cu) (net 7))
 (segment (start 156.672 138.6626) (end 155.5536 139.781) (width 0.2) (layer B.Cu) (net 7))
 (segment (start 155.5536 139.781) (end 152.481 139.781) (width 0.2) (layer B.Cu) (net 7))
 (segment (start 152.481 139.781) (end 151.13 138.43) (width 0.2) (layer B.Cu) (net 7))
 (segment (start 149.86 87.07) (end 149.86 87.7703) (width 0.2) (layer F.Cu) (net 8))
 (segment (start 149.86 129.54) (end 149.86 128.8397) (width 0.2) (layer F.Cu) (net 8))
 (segment (start 149.86 128.8397) (end 149.8904 128.8093) (width 0.2) (layer F.Cu) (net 8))
 (segment (start 149.8904 128.8093) (end 149.8904 87.8007) (width 0.2) (layer F.Cu) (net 8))
 (segment (start 149.8904 87.8007) (end 149.86 87.7703) (width 0.2) (layer F.Cu) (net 8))
 (segment (start 149.86 138.43) (end 149.0942 137.6642) (width 0.2) (layer F.Cu) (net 8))
 (segment (start 149.0942 137.6642) (end 149.0942 130.3058) (width 0.2) (layer F.Cu) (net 8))
 (segment (start 149.0942 130.3058) (end 149.86 129.54) (width 0.2) (layer F.Cu) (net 8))
 (segment (start 152.4 114.75) (end 148.59 118.56) (width 0.2) (layer B.Cu) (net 9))
 (segment (start 148.59 118.56) (end 148.59 120.65) (width 0.2) (layer B.Cu) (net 9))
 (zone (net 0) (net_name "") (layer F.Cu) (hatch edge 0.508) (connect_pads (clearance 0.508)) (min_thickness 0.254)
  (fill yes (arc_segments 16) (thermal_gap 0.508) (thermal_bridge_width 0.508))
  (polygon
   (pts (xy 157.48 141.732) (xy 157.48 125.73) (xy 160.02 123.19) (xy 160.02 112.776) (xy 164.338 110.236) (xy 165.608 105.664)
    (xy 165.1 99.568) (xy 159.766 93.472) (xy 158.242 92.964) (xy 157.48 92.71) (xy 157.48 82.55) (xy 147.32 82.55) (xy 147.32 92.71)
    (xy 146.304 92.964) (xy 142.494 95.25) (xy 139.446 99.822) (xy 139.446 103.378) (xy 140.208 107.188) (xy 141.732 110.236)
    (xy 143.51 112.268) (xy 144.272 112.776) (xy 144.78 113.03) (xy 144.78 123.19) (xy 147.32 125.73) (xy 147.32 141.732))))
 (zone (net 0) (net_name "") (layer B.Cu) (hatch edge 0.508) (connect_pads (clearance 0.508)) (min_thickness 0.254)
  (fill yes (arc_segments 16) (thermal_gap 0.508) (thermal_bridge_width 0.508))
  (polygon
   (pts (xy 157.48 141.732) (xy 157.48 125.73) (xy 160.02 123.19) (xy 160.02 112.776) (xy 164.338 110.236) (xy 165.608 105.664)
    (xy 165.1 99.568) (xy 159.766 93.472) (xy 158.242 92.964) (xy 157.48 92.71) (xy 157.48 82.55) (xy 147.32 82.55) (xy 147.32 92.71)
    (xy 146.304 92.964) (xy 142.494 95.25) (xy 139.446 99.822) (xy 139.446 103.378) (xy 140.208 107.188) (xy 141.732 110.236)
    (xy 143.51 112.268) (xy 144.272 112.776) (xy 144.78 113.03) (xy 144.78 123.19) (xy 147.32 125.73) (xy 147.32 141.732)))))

